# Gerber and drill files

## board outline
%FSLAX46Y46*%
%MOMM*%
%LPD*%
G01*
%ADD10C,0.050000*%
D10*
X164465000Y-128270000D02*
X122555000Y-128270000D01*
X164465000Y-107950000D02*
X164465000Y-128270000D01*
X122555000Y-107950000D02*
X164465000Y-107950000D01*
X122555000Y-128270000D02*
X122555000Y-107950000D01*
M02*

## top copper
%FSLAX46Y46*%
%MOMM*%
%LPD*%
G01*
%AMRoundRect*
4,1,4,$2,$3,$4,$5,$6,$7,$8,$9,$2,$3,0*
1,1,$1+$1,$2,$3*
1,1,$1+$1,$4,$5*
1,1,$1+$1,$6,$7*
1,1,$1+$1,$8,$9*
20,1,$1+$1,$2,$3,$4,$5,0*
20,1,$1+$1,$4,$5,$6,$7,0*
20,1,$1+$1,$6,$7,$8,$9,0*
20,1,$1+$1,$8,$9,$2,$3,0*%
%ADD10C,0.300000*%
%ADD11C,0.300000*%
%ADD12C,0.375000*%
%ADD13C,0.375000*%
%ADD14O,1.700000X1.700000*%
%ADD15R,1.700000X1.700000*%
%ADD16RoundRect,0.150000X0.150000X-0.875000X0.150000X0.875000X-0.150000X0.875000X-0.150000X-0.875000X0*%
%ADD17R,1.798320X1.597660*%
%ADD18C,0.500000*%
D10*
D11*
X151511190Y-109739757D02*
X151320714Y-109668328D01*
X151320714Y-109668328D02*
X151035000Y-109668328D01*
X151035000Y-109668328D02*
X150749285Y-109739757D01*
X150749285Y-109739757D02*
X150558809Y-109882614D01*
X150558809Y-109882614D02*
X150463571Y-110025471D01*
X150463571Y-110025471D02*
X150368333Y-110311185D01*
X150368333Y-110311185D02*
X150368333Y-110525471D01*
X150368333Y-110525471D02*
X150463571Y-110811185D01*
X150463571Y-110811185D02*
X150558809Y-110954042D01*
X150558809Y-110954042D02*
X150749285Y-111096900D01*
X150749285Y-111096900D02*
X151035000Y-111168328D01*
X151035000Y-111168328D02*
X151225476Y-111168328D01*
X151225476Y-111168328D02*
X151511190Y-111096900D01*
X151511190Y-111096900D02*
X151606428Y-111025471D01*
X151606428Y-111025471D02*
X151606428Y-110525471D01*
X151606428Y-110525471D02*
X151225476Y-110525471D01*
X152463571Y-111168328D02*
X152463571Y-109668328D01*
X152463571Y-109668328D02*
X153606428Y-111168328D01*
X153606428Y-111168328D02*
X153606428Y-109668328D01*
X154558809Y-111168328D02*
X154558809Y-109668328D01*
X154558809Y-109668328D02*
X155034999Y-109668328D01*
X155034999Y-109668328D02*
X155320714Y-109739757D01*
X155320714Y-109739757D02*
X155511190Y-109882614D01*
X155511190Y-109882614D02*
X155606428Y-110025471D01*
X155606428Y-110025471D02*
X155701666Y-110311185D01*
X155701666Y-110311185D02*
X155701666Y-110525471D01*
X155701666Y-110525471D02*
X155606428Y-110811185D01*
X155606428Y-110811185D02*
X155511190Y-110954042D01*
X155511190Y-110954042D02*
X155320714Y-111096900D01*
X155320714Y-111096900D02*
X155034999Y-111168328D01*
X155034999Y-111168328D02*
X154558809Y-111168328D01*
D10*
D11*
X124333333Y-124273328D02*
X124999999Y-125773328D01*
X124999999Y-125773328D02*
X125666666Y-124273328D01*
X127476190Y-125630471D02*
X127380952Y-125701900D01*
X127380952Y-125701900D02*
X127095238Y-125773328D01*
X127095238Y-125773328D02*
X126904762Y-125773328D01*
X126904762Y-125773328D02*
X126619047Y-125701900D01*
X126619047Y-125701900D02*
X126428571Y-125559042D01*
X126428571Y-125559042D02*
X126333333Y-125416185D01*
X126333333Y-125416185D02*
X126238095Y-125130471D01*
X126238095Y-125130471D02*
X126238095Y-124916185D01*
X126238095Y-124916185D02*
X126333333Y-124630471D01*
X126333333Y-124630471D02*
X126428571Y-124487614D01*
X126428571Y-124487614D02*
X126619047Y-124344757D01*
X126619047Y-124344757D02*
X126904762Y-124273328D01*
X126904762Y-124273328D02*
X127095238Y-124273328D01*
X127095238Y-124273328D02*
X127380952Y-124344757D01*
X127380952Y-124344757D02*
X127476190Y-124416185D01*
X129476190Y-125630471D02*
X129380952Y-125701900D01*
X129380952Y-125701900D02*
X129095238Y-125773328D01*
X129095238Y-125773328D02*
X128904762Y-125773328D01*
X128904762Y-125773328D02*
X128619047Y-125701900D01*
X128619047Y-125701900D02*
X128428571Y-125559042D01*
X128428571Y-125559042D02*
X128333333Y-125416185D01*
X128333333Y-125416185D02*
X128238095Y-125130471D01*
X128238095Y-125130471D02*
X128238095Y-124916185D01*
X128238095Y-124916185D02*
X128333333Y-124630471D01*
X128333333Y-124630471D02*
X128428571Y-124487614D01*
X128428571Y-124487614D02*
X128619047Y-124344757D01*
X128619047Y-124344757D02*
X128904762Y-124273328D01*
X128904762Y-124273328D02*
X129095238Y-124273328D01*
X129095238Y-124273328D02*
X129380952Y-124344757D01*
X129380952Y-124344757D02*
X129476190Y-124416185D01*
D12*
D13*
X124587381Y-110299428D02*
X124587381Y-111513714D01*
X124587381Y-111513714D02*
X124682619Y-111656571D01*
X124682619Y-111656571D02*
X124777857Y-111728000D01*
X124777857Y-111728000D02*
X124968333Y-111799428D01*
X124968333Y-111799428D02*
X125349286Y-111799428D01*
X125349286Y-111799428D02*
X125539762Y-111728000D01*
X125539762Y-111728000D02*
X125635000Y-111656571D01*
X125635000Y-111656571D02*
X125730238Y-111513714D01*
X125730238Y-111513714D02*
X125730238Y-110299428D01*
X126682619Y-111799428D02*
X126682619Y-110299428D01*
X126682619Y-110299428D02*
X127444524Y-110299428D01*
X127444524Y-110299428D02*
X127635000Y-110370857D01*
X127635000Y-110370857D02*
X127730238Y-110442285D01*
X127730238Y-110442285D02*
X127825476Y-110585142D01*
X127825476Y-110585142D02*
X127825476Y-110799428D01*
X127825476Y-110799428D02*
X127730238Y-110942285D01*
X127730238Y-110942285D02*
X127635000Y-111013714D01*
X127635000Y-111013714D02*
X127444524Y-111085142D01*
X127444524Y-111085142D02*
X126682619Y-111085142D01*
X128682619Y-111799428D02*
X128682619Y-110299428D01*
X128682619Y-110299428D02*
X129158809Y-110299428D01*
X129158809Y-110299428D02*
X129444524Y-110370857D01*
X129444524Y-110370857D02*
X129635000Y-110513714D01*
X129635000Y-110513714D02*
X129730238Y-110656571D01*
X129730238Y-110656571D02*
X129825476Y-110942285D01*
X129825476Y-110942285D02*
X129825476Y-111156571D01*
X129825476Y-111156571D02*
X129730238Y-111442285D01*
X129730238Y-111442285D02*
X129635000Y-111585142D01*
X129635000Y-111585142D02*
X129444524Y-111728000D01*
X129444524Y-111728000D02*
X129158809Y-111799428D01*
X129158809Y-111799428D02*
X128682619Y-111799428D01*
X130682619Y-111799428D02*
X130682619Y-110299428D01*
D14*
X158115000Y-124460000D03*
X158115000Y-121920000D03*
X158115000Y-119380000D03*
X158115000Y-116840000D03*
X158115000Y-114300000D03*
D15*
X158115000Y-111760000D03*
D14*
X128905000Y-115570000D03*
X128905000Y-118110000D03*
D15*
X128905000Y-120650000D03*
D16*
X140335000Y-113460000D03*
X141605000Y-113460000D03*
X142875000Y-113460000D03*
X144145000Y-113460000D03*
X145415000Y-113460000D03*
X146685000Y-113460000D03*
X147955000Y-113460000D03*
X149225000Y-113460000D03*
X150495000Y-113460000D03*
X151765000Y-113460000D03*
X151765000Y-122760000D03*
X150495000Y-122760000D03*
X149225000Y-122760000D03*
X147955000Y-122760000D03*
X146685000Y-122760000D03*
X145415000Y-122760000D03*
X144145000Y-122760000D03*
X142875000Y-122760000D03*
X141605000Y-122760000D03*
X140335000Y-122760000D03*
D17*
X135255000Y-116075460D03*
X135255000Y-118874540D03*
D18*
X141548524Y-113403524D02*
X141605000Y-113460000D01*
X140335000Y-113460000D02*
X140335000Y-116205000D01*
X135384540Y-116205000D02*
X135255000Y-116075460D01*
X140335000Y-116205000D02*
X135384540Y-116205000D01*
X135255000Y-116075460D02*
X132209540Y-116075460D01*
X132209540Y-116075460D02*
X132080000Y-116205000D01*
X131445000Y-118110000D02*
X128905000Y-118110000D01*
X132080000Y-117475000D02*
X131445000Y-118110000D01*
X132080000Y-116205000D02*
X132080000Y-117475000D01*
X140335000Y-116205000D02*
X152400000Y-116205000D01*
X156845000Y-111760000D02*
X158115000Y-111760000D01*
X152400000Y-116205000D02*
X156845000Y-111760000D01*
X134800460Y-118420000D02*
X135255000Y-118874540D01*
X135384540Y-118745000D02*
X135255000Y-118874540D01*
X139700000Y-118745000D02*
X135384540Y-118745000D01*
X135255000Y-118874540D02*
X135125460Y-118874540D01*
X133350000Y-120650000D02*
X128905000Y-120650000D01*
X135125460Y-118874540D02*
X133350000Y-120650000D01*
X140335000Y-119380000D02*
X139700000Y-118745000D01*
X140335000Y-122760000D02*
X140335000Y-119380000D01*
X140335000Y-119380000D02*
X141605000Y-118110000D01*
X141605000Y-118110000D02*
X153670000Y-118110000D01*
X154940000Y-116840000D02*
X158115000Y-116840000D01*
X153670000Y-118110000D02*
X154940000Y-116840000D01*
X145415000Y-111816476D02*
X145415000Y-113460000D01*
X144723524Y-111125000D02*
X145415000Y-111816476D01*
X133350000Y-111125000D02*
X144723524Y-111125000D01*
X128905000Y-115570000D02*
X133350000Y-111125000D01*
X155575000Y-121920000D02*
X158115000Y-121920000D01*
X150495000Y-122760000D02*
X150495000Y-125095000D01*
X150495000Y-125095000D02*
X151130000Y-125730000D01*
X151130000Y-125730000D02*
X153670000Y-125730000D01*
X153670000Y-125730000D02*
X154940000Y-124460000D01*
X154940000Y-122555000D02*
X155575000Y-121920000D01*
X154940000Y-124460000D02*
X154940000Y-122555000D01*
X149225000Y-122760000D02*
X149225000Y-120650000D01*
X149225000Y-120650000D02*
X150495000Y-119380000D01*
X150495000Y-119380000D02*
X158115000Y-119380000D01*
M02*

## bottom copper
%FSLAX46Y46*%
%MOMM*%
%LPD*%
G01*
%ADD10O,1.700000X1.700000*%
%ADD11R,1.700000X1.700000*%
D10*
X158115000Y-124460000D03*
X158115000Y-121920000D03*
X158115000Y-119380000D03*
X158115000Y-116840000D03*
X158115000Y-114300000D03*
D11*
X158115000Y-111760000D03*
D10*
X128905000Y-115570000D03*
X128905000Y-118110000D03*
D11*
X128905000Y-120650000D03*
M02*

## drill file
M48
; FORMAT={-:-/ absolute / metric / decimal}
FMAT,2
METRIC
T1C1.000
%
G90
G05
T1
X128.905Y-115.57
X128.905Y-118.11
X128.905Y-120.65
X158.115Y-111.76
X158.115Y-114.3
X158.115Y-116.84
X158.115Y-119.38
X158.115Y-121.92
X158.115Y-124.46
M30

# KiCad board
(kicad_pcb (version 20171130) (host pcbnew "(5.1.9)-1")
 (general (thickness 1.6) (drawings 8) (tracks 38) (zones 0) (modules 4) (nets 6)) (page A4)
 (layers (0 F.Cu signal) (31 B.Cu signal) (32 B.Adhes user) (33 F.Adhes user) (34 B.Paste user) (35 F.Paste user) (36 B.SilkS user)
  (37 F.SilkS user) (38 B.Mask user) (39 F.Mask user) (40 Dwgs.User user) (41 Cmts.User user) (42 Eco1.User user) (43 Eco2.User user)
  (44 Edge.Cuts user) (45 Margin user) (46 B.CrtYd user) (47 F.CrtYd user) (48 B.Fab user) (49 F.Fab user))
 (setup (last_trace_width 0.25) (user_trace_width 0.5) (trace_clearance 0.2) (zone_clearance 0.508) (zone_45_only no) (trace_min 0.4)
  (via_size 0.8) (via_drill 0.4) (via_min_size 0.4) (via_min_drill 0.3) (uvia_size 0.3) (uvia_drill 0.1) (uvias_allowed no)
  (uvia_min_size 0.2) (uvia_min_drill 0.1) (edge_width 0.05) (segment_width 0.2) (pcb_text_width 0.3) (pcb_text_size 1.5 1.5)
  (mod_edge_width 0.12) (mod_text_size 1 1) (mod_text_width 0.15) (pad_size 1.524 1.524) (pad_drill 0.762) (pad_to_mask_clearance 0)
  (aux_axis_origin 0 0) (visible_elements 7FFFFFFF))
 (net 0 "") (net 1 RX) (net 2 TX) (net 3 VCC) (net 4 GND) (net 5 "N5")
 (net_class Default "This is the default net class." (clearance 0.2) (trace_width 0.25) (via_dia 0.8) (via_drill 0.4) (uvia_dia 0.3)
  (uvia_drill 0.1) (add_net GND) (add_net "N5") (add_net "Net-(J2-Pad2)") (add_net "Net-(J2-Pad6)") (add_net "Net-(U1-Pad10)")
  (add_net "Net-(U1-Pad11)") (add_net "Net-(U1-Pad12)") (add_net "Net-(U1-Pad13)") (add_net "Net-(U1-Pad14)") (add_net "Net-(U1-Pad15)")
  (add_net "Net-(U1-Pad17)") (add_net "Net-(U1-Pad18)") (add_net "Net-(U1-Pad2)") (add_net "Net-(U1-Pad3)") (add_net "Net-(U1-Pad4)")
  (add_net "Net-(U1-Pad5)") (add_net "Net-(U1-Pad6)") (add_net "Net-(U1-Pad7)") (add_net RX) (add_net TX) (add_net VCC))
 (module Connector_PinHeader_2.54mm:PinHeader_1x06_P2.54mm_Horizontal (layer F.Cu) (at 158.115 111.76)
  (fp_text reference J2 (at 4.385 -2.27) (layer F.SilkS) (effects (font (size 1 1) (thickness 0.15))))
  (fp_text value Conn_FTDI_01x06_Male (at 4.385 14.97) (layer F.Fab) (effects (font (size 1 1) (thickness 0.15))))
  (pad 6 thru_hole oval (at 0 12.7) (size 1.7 1.7) (drill 1) (layers *.Cu *.Mask))
  (pad 5 thru_hole oval (at 0 10.16) (size 1.7 1.7) (drill 1) (layers *.Cu *.Mask) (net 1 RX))
  (pad 4 thru_hole oval (at 0 7.62) (size 1.7 1.7) (drill 1) (layers *.Cu *.Mask) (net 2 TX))
  (pad 3 thru_hole oval (at 0 5.08) (size 1.7 1.7) (drill 1) (layers *.Cu *.Mask) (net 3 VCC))
  (pad 2 thru_hole oval (at 0 2.54) (size 1.7 1.7) (drill 1) (layers *.Cu *.Mask))
  (pad 1 thru_hole rect (at 0 0) (size 1.7 1.7) (drill 1) (layers *.Cu *.Mask) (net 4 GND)))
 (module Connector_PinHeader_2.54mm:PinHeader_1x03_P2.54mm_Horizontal (layer F.Cu) (at 128.905 120.65 180)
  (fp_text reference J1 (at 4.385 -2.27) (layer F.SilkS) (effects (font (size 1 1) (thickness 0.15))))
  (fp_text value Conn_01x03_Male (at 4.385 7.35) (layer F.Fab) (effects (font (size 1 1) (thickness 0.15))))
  (pad 3 thru_hole oval (at 0 5.08 180) (size 1.7 1.7) (drill 1) (layers *.Cu *.Mask) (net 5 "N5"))
  (pad 2 thru_hole oval (at 0 2.54 180) (size 1.7 1.7) (drill 1) (layers *.Cu *.Mask) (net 4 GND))
  (pad 1 thru_hole rect (at 0 0 180) (size 1.7 1.7) (drill 1) (layers *.Cu *.Mask) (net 3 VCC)))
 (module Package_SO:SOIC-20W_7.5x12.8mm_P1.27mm (layer F.Cu) (at 146.05 118.11 90)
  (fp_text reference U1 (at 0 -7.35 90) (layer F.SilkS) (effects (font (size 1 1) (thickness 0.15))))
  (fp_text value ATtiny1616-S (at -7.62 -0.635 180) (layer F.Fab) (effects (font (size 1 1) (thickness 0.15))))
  (pad 20 smd roundrect (at 4.65 -5.715 90) (size 2.05 0.6) (layers F.Cu F.Paste F.Mask) (roundrect_rratio 0.25) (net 4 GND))
  (pad 19 smd roundrect (at 4.65 -4.445 90) (size 2.05 0.6) (layers F.Cu F.Paste F.Mask) (roundrect_rratio 0.25))
  (pad 18 smd roundrect (at 4.65 -3.175 90) (size 2.05 0.6) (layers F.Cu F.Paste F.Mask) (roundrect_rratio 0.25))
  (pad 17 smd roundrect (at 4.65 -1.905 90) (size 2.05 0.6) (layers F.Cu F.Paste F.Mask) (roundrect_rratio 0.25))
  (pad 16 smd roundrect (at 4.65 -0.635 90) (size 2.05 0.6) (layers F.Cu F.Paste F.Mask) (roundrect_rratio 0.25) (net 5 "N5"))
  (pad 15 smd roundrect (at 4.65 0.635 90) (size 2.05 0.6) (layers F.Cu F.Paste F.Mask) (roundrect_rratio 0.25))
  (pad 14 smd roundrect (at 4.65 1.905 90) (size 2.05 0.6) (layers F.Cu F.Paste F.Mask) (roundrect_rratio 0.25))
  (pad 13 smd roundrect (at 4.65 3.175 90) (size 2.05 0.6) (layers F.Cu F.Paste F.Mask) (roundrect_rratio 0.25))
  (pad 12 smd roundrect (at 4.65 4.445 90) (size 2.05 0.6) (layers F.Cu F.Paste F.Mask) (roundrect_rratio 0.25))
  (pad 11 smd roundrect (at 4.65 5.715 90) (size 2.05 0.6) (layers F.Cu F.Paste F.Mask) (roundrect_rratio 0.25))
  (pad 10 smd roundrect (at -4.65 5.715 90) (size 2.05 0.6) (layers F.Cu F.Paste F.Mask) (roundrect_rratio 0.25))
  (pad 9 smd roundrect (at -4.65 4.445 90) (size 2.05 0.6) (layers F.Cu F.Paste F.Mask) (roundrect_rratio 0.25) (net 1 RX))
  (pad 8 smd roundrect (at -4.65 3.175 90) (size 2.05 0.6) (layers F.Cu F.Paste F.Mask) (roundrect_rratio 0.25) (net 2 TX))
  (pad 7 smd roundrect (at -4.65 1.905 90) (size 2.05 0.6) (layers F.Cu F.Paste F.Mask) (roundrect_rratio 0.25))
  (pad 6 smd roundrect (at -4.65 0.635 90) (size 2.05 0.6) (layers F.Cu F.Paste F.Mask) (roundrect_rratio 0.25))
  (pad 5 smd roundrect (at -4.65 -0.635 90) (size 2.05 0.6) (layers F.Cu F.Paste F.Mask) (roundrect_rratio 0.25))
  (pad 4 smd roundrect (at -4.65 -1.905 90) (size 2.05 0.6) (layers F.Cu F.Paste F.Mask) (roundrect_rratio 0.25))
  (pad 3 smd roundrect (at -4.65 -3.175 90) (size 2.05 0.6) (layers F.Cu F.Paste F.Mask) (roundrect_rratio 0.25))
  (pad 2 smd roundrect (at -4.65 -4.445 90) (size 2.05 0.6) (layers F.Cu F.Paste F.Mask) (roundrect_rratio 0.25))
  (pad 1 smd roundrect (at -4.65 -5.715 90) (size 2.05 0.6) (layers F.Cu F.Paste F.Mask) (roundrect_rratio 0.25) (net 3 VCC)))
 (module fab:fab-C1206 (layer F.Cu) (at 135.255 117.475 90)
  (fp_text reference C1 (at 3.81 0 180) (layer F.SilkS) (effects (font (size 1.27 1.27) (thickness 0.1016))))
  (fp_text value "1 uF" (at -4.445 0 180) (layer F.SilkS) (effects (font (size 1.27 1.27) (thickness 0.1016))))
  (pad 2 smd rect (at 1.39954 0 90) (size 1.59766 1.79832) (layers F.Cu F.Paste F.Mask) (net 4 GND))
  (pad 1 smd rect (at -1.39954 0 90) (size 1.59766 1.79832) (layers F.Cu F.Paste F.Mask) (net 3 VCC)))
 (gr_line (start 164.465 128.27) (end 122.555 128.27) (layer Edge.Cuts) (width 0.05))
 (gr_line (start 164.465 107.95) (end 164.465 128.27) (layer Edge.Cuts) (width 0.05))
 (gr_line (start 122.555 107.95) (end 164.465 107.95) (layer Edge.Cuts) (width 0.05))
 (gr_line (start 122.555 128.27) (end 122.555 107.95) (layer Edge.Cuts) (width 0.05))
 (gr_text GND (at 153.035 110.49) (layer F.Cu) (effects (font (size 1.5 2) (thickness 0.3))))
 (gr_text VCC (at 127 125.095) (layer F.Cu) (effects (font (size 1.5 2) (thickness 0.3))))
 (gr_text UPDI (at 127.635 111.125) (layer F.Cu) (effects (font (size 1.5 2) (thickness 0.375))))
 (segment (start 141.548524 113.403524) (end 141.605 113.46) (width 0.5) (layer F.Cu) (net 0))
 (segment (start 140.335 113.46) (end 140.335 116.205) (width 0.5) (layer F.Cu) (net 4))
 (segment (start 135.38454 116.205) (end 135.255 116.07546) (width 0.5) (layer F.Cu) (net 4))
 (segment (start 140.335 116.205) (end 135.38454 116.205) (width 0.5) (layer F.Cu) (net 4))
 (segment (start 135.255 116.07546) (end 132.20954 116.07546) (width 0.5) (layer F.Cu) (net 4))
 (segment (start 132.20954 116.07546) (end 132.08 116.205) (width 0.5) (layer F.Cu) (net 4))
 (segment (start 131.445 118.11) (end 128.905 118.11) (width 0.5) (layer F.Cu) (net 4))
 (segment (start 132.08 117.475) (end 131.445 118.11) (width 0.5) (layer F.Cu) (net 4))
 (segment (start 132.08 116.205) (end 132.08 117.475) (width 0.5) (layer F.Cu) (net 4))
 (segment (start 140.335 116.205) (end 152.4 116.205) (width 0.5) (layer F.Cu) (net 4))
 (segment (start 156.845 111.76) (end 158.115 111.76) (width 0.5) (layer F.Cu) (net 4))
 (segment (start 152.4 116.205) (end 156.845 111.76) (width 0.5) (layer F.Cu) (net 4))
 (segment (start 134.80046 118.42) (end 135.255 118.87454) (width 0.5) (layer F.Cu) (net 3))
 (segment (start 135.38454 118.745) (end 135.255 118.87454) (width 0.5) (layer F.Cu) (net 3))
 (segment (start 139.7 118.745) (end 135.38454 118.745) (width 0.5) (layer F.Cu) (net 3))
 (segment (start 135.255 118.87454) (end 135.12546 118.87454) (width 0.5) (layer F.Cu) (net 3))
 (segment (start 133.35 120.65) (end 128.905 120.65) (width 0.5) (layer F.Cu) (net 3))
 (segment (start 135.12546 118.87454) (end 133.35 120.65) (width 0.5) (layer F.Cu) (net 3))
 (segment (start 140.335 119.38) (end 139.7 118.745) (width 0.5) (layer F.Cu) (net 3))
 (segment (start 140.335 122.76) (end 140.335 119.38) (width 0.5) (layer F.Cu) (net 3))
 (segment (start 140.335 119.38) (end 141.605 118.11) (width 0.5) (layer F.Cu) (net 3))
 (segment (start 141.605 118.11) (end 153.67 118.11) (width 0.5) (layer F.Cu) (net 3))
 (segment (start 154.94 116.84) (end 158.115 116.84) (width 0.5) (layer F.Cu) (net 3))
 (segment (start 153.67 118.11) (end 154.94 116.84) (width 0.5) (layer F.Cu) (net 3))
 (segment (start 145.415 111.816476) (end 145.415 113.46) (width 0.5) (layer F.Cu) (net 5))
 (segment (start 144.723524 111.125) (end 145.415 111.816476) (width 0.5) (layer F.Cu) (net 5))
 (segment (start 133.35 111.125) (end 144.723524 111.125) (width 0.5) (layer F.Cu) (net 5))
 (segment (start 128.905 115.57) (end 133.35 111.125) (width 0.5) (layer F.Cu) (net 5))
 (segment (start 155.575 121.92) (end 158.115 121.92) (width 0.5) (layer F.Cu) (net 1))
 (segment (start 150.495 122.76) (end 150.495 125.095) (width 0.5) (layer F.Cu) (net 1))
 (segment (start 150.495 125.095) (end 151.13 125.73) (width 0.5) (layer F.Cu) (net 1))
 (segment (start 151.13 125.73) (end 153.67 125.73) (width 0.5) (layer F.Cu) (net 1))
 (segment (start 153.67 125.73) (end 154.94 124.46) (width 0.5) (layer F.Cu) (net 1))
 (segment (start 154.94 122.555) (end 155.575 121.92) (width 0.5) (layer F.Cu) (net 1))
 (segment (start 154.94 124.46) (end 154.94 122.555) (width 0.5) (layer F.Cu) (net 1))
 (segment (start 149.225 122.76) (end 149.225 120.65) (width 0.5) (layer F.Cu) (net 2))
 (segment (start 149.225 120.65) (end 150.495 119.38) (width 0.5) (layer F.Cu) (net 2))
 (segment (start 150.495 119.38) (end 158.115 119.38) (width 0.5) (layer F.Cu) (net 2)))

